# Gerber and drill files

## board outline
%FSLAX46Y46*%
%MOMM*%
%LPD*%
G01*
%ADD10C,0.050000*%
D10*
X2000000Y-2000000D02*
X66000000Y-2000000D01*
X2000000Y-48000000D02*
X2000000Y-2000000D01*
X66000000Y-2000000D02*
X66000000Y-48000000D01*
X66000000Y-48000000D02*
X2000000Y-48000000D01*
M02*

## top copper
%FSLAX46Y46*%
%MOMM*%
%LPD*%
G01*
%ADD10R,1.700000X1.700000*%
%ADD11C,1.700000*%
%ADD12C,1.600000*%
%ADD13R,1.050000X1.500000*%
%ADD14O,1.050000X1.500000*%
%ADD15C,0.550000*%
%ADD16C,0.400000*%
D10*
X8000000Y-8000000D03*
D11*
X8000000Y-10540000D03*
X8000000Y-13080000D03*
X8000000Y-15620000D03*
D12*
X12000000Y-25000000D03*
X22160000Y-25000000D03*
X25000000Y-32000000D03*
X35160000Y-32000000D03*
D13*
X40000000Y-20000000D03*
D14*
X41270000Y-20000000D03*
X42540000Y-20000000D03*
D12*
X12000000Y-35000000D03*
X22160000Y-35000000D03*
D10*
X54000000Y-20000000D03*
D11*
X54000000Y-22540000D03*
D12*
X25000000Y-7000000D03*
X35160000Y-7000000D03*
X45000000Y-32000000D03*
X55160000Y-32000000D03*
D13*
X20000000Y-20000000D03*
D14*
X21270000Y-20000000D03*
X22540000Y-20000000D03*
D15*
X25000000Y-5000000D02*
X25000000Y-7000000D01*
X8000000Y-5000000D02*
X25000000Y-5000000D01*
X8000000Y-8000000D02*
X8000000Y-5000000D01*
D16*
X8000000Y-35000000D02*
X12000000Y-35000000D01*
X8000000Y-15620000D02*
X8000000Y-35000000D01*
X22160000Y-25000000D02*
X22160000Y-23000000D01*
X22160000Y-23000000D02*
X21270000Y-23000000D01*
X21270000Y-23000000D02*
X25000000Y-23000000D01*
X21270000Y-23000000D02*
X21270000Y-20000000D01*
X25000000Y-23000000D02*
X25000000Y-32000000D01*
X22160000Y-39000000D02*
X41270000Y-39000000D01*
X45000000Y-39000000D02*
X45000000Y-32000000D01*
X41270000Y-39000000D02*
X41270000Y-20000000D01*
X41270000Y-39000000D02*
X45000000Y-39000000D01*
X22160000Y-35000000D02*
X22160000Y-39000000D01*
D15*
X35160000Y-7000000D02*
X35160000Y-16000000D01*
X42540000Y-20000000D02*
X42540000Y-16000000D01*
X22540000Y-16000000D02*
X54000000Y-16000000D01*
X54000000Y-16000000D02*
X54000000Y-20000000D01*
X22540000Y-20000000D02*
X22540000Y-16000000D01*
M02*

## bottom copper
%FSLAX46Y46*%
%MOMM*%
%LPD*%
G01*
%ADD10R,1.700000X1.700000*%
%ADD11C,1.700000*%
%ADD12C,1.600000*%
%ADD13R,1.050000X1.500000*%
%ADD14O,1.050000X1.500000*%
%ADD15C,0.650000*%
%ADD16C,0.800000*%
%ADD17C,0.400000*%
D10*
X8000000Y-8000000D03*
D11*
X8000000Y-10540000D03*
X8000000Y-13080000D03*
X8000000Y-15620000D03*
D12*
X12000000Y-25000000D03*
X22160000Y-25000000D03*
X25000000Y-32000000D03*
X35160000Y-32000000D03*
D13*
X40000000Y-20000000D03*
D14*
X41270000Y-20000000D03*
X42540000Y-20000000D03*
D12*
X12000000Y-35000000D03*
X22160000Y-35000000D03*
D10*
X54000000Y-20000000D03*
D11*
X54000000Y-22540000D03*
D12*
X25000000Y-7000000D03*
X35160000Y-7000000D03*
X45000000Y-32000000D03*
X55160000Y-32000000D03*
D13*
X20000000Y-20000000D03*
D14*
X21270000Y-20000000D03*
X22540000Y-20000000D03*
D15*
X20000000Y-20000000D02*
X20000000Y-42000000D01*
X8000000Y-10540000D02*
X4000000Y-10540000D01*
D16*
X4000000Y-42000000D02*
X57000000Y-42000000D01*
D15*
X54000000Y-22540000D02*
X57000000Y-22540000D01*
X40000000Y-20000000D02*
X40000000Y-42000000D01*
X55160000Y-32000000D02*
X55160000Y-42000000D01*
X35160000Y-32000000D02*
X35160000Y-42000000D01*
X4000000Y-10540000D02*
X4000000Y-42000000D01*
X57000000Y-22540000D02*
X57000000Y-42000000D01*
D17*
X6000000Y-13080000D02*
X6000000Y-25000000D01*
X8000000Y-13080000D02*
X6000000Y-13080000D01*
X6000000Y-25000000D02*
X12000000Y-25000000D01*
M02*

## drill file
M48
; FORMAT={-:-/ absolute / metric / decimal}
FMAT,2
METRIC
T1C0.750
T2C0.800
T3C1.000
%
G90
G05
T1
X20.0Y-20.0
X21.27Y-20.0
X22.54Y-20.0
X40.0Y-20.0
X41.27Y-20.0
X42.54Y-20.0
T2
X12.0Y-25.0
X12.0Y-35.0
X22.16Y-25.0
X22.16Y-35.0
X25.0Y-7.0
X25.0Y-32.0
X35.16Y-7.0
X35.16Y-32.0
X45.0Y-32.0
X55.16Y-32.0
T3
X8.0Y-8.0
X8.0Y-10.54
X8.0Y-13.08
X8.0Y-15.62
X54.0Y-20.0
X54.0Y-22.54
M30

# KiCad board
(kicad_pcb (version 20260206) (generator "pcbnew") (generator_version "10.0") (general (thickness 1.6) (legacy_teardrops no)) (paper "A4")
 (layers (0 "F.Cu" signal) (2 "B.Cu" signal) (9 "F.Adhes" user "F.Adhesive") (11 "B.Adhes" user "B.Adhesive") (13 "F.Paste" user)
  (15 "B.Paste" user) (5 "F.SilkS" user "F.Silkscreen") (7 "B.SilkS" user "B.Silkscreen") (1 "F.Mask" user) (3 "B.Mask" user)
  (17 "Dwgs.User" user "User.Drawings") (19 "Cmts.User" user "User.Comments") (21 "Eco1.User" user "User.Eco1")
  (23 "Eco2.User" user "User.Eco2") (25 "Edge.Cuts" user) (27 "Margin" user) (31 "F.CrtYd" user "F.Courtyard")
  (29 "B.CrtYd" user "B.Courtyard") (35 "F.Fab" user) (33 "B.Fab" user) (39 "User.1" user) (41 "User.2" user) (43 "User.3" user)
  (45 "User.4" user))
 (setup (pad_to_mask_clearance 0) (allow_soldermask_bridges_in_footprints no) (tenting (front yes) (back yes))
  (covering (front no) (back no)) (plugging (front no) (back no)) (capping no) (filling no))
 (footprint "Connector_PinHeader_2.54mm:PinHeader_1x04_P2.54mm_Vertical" (layer "F.Cu") (at 8 8)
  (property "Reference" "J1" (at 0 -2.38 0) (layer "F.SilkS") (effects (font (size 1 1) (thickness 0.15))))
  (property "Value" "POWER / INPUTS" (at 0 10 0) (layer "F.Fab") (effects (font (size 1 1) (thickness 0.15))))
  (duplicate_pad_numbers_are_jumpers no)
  (pad "1" thru_hole rect (at 0 0) (size 1.7 1.7) (drill 1) (layers "*.Cu" "*.Mask") (remove_unused_layers no) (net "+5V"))
  (pad "2" thru_hole circle (at 0 2.54) (size 1.7 1.7) (drill 1) (layers "*.Cu" "*.Mask") (remove_unused_layers no) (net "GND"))
  (pad "3" thru_hole circle (at 0 5.08) (size 1.7 1.7) (drill 1) (layers "*.Cu" "*.Mask") (remove_unused_layers no) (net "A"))
  (pad "4" thru_hole circle (at 0 7.62) (size 1.7 1.7) (drill 1) (layers "*.Cu" "*.Mask") (remove_unused_layers no) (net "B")))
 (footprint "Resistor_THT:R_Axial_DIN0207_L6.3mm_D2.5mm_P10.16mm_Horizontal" (layer "F.Cu") (at 12 25)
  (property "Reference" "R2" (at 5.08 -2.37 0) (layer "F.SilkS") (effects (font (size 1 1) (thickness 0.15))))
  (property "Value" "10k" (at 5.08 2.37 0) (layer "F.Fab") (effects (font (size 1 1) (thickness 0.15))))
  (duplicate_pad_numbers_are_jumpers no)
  (pad "1" thru_hole circle (at 0 0) (size 1.6 1.6) (drill 0.8) (layers "*.Cu" "*.Mask") (remove_unused_layers no) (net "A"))
  (pad "2" thru_hole circle (at 10.16 0) (size 1.6 1.6) (drill 0.8) (layers "*.Cu" "*.Mask") (remove_unused_layers no) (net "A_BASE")))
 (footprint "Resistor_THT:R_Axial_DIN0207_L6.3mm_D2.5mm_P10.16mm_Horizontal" (layer "F.Cu") (at 25 32)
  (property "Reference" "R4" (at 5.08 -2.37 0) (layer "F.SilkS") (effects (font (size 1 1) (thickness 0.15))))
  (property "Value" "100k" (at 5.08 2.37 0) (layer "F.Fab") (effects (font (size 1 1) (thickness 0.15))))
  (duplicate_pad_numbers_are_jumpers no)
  (pad "1" thru_hole circle (at 0 0) (size 1.6 1.6) (drill 0.8) (layers "*.Cu" "*.Mask") (remove_unused_layers no) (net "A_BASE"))
  (pad "2" thru_hole circle (at 10.16 0) (size 1.6 1.6) (drill 0.8) (layers "*.Cu" "*.Mask") (remove_unused_layers no) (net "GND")))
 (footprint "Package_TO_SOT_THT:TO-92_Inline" (layer "F.Cu") (at 40 20)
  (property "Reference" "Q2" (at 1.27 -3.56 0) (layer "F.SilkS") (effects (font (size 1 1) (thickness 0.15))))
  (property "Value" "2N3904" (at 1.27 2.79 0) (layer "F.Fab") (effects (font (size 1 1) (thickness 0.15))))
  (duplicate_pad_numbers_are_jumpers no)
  (pad "1" thru_hole rect (at 0 0) (size 1.05 1.5) (drill 0.75) (layers "*.Cu" "*.Mask") (remove_unused_layers no) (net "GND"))
  (pad "2" thru_hole oval (at 1.27 0) (size 1.05 1.5) (drill 0.75) (layers "*.Cu" "*.Mask") (remove_unused_layers no) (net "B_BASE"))
  (pad "3" thru_hole oval (at 2.54 0) (size 1.05 1.5) (drill 0.75) (layers "*.Cu" "*.Mask") (remove_unused_layers no) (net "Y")))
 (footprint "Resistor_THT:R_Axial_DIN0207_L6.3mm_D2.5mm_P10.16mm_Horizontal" (layer "F.Cu") (at 12 35)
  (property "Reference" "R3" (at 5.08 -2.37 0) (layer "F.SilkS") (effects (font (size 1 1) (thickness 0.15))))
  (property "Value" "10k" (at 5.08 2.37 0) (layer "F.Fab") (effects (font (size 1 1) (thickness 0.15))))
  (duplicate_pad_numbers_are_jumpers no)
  (pad "1" thru_hole circle (at 0 0) (size 1.6 1.6) (drill 0.8) (layers "*.Cu" "*.Mask") (remove_unused_layers no) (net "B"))
  (pad "2" thru_hole circle (at 10.16 0) (size 1.6 1.6) (drill 0.8) (layers "*.Cu" "*.Mask") (remove_unused_layers no) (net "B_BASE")))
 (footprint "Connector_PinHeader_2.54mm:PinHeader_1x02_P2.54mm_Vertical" (layer "F.Cu") (at 54 20)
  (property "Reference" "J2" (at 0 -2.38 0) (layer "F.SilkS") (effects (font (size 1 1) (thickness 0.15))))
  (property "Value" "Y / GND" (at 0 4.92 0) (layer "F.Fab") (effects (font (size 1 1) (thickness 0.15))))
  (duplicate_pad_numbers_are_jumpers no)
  (pad "1" thru_hole rect (at 0 0) (size 1.7 1.7) (drill 1) (layers "*.Cu" "*.Mask") (remove_unused_layers no) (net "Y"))
  (pad "2" thru_hole circle (at 0 2.54) (size 1.7 1.7) (drill 1) (layers "*.Cu" "*.Mask") (remove_unused_layers no) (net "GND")))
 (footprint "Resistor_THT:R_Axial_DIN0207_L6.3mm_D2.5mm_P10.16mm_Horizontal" (layer "F.Cu") (at 25 7)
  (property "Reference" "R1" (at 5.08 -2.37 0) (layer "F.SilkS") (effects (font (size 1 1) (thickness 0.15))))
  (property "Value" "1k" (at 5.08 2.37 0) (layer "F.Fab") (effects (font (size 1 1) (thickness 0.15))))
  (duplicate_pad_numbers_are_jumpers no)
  (pad "1" thru_hole circle (at 0 0) (size 1.6 1.6) (drill 0.8) (layers "*.Cu" "*.Mask") (remove_unused_layers no) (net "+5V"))
  (pad "2" thru_hole circle (at 10.16 0) (size 1.6 1.6) (drill 0.8) (layers "*.Cu" "*.Mask") (remove_unused_layers no) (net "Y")))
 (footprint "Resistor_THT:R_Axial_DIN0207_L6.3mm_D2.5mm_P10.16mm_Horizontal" (layer "F.Cu") (at 45 32)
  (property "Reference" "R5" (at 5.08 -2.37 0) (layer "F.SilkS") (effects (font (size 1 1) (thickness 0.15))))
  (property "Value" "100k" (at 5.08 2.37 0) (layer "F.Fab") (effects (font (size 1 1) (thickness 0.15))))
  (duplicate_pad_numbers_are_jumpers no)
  (pad "1" thru_hole circle (at 0 0) (size 1.6 1.6) (drill 0.8) (layers "*.Cu" "*.Mask") (remove_unused_layers no) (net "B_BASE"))
  (pad "2" thru_hole circle (at 10.16 0) (size 1.6 1.6) (drill 0.8) (layers "*.Cu" "*.Mask") (remove_unused_layers no) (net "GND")))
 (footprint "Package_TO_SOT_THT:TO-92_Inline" (layer "F.Cu") (at 20 20)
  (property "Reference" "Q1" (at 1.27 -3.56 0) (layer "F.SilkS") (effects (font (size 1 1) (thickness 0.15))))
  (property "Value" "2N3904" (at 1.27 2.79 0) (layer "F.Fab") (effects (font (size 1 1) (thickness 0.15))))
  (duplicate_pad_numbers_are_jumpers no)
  (pad "1" thru_hole rect (at 0 0) (size 1.05 1.5) (drill 0.75) (layers "*.Cu" "*.Mask") (remove_unused_layers no) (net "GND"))
  (pad "2" thru_hole oval (at 1.27 0) (size 1.05 1.5) (drill 0.75) (layers "*.Cu" "*.Mask") (remove_unused_layers no) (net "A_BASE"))
  (pad "3" thru_hole oval (at 2.54 0) (size 1.05 1.5) (drill 0.75) (layers "*.Cu" "*.Mask") (remove_unused_layers no) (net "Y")))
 (gr_line (start 2 2) (end 66 2) (stroke (width 0.05) (type default)) (layer "Edge.Cuts"))
 (gr_line (start 2 48) (end 2 2) (stroke (width 0.05) (type default)) (layer "Edge.Cuts"))
 (gr_line (start 66 2) (end 66 48) (stroke (width 0.05) (type default)) (layer "Edge.Cuts"))
 (gr_line (start 66 48) (end 2 48) (stroke (width 0.05) (type default)) (layer "Edge.Cuts"))
 (segment (start 25 5) (end 25 7) (width 0.55) (layer "F.Cu") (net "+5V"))
 (segment (start 8 5) (end 25 5) (width 0.55) (layer "F.Cu") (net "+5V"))
 (segment (start 8 8) (end 8 5) (width 0.55) (layer "F.Cu") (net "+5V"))
 (segment (start 20 20) (end 20 42) (width 0.65) (layer "B.Cu") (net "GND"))
 (segment (start 8 10.54) (end 4 10.54) (width 0.65) (layer "B.Cu") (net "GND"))
 (segment (start 4 42) (end 57 42) (width 0.8) (layer "B.Cu") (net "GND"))
 (segment (start 54 22.54) (end 57 22.54) (width 0.65) (layer "B.Cu") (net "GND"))
 (segment (start 40 20) (end 40 42) (width 0.65) (layer "B.Cu") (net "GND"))
 (segment (start 55.16 32) (end 55.16 42) (width 0.65) (layer "B.Cu") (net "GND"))
 (segment (start 35.16 32) (end 35.16 42) (width 0.65) (layer "B.Cu") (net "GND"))
 (segment (start 4 10.54) (end 4 42) (width 0.65) (layer "B.Cu") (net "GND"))
 (segment (start 57 22.54) (end 57 42) (width 0.65) (layer "B.Cu") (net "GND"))
 (segment (start 6 13.08) (end 6 25) (width 0.4) (layer "B.Cu") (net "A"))
 (segment (start 8 13.08) (end 6 13.08) (width 0.4) (layer "B.Cu") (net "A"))
 (segment (start 6 25) (end 12 25) (width 0.4) (layer "B.Cu") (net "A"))
 (segment (start 8 35) (end 12 35) (width 0.4) (layer "F.Cu") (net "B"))
 (segment (start 8 15.62) (end 8 35) (width 0.4) (layer "F.Cu") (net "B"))
 (segment (start 22.16 25) (end 22.16 23) (width 0.4) (layer "F.Cu") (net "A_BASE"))
 (segment (start 22.16 23) (end 21.27 23) (width 0.4) (layer "F.Cu") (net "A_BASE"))
 (segment (start 21.27 23) (end 25 23) (width 0.4) (layer "F.Cu") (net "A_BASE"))
 (segment (start 21.27 23) (end 21.27 20) (width 0.4) (layer "F.Cu") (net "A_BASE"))
 (segment (start 25 23) (end 25 32) (width 0.4) (layer "F.Cu") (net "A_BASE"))
 (segment (start 22.16 39) (end 41.27 39) (width 0.4) (layer "F.Cu") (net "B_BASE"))
 (segment (start 45 39) (end 45 32) (width 0.4) (layer "F.Cu") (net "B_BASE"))
 (segment (start 41.27 39) (end 41.27 20) (width 0.4) (layer "F.Cu") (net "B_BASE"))
 (segment (start 41.27 39) (end 45 39) (width 0.4) (layer "F.Cu") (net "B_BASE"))
 (segment (start 22.16 35) (end 22.16 39) (width 0.4) (layer "F.Cu") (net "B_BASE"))
 (segment (start 35.16 7) (end 35.16 16) (width 0.55) (layer "F.Cu") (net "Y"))
 (segment (start 42.54 20) (end 42.54 16) (width 0.55) (layer "F.Cu") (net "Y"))
 (segment (start 22.54 16) (end 54 16) (width 0.55) (layer "F.Cu") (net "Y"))
 (segment (start 54 16) (end 54 20) (width 0.55) (layer "F.Cu") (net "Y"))
 (segment (start 22.54 20) (end 22.54 16) (width 0.55) (layer "F.Cu") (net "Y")))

